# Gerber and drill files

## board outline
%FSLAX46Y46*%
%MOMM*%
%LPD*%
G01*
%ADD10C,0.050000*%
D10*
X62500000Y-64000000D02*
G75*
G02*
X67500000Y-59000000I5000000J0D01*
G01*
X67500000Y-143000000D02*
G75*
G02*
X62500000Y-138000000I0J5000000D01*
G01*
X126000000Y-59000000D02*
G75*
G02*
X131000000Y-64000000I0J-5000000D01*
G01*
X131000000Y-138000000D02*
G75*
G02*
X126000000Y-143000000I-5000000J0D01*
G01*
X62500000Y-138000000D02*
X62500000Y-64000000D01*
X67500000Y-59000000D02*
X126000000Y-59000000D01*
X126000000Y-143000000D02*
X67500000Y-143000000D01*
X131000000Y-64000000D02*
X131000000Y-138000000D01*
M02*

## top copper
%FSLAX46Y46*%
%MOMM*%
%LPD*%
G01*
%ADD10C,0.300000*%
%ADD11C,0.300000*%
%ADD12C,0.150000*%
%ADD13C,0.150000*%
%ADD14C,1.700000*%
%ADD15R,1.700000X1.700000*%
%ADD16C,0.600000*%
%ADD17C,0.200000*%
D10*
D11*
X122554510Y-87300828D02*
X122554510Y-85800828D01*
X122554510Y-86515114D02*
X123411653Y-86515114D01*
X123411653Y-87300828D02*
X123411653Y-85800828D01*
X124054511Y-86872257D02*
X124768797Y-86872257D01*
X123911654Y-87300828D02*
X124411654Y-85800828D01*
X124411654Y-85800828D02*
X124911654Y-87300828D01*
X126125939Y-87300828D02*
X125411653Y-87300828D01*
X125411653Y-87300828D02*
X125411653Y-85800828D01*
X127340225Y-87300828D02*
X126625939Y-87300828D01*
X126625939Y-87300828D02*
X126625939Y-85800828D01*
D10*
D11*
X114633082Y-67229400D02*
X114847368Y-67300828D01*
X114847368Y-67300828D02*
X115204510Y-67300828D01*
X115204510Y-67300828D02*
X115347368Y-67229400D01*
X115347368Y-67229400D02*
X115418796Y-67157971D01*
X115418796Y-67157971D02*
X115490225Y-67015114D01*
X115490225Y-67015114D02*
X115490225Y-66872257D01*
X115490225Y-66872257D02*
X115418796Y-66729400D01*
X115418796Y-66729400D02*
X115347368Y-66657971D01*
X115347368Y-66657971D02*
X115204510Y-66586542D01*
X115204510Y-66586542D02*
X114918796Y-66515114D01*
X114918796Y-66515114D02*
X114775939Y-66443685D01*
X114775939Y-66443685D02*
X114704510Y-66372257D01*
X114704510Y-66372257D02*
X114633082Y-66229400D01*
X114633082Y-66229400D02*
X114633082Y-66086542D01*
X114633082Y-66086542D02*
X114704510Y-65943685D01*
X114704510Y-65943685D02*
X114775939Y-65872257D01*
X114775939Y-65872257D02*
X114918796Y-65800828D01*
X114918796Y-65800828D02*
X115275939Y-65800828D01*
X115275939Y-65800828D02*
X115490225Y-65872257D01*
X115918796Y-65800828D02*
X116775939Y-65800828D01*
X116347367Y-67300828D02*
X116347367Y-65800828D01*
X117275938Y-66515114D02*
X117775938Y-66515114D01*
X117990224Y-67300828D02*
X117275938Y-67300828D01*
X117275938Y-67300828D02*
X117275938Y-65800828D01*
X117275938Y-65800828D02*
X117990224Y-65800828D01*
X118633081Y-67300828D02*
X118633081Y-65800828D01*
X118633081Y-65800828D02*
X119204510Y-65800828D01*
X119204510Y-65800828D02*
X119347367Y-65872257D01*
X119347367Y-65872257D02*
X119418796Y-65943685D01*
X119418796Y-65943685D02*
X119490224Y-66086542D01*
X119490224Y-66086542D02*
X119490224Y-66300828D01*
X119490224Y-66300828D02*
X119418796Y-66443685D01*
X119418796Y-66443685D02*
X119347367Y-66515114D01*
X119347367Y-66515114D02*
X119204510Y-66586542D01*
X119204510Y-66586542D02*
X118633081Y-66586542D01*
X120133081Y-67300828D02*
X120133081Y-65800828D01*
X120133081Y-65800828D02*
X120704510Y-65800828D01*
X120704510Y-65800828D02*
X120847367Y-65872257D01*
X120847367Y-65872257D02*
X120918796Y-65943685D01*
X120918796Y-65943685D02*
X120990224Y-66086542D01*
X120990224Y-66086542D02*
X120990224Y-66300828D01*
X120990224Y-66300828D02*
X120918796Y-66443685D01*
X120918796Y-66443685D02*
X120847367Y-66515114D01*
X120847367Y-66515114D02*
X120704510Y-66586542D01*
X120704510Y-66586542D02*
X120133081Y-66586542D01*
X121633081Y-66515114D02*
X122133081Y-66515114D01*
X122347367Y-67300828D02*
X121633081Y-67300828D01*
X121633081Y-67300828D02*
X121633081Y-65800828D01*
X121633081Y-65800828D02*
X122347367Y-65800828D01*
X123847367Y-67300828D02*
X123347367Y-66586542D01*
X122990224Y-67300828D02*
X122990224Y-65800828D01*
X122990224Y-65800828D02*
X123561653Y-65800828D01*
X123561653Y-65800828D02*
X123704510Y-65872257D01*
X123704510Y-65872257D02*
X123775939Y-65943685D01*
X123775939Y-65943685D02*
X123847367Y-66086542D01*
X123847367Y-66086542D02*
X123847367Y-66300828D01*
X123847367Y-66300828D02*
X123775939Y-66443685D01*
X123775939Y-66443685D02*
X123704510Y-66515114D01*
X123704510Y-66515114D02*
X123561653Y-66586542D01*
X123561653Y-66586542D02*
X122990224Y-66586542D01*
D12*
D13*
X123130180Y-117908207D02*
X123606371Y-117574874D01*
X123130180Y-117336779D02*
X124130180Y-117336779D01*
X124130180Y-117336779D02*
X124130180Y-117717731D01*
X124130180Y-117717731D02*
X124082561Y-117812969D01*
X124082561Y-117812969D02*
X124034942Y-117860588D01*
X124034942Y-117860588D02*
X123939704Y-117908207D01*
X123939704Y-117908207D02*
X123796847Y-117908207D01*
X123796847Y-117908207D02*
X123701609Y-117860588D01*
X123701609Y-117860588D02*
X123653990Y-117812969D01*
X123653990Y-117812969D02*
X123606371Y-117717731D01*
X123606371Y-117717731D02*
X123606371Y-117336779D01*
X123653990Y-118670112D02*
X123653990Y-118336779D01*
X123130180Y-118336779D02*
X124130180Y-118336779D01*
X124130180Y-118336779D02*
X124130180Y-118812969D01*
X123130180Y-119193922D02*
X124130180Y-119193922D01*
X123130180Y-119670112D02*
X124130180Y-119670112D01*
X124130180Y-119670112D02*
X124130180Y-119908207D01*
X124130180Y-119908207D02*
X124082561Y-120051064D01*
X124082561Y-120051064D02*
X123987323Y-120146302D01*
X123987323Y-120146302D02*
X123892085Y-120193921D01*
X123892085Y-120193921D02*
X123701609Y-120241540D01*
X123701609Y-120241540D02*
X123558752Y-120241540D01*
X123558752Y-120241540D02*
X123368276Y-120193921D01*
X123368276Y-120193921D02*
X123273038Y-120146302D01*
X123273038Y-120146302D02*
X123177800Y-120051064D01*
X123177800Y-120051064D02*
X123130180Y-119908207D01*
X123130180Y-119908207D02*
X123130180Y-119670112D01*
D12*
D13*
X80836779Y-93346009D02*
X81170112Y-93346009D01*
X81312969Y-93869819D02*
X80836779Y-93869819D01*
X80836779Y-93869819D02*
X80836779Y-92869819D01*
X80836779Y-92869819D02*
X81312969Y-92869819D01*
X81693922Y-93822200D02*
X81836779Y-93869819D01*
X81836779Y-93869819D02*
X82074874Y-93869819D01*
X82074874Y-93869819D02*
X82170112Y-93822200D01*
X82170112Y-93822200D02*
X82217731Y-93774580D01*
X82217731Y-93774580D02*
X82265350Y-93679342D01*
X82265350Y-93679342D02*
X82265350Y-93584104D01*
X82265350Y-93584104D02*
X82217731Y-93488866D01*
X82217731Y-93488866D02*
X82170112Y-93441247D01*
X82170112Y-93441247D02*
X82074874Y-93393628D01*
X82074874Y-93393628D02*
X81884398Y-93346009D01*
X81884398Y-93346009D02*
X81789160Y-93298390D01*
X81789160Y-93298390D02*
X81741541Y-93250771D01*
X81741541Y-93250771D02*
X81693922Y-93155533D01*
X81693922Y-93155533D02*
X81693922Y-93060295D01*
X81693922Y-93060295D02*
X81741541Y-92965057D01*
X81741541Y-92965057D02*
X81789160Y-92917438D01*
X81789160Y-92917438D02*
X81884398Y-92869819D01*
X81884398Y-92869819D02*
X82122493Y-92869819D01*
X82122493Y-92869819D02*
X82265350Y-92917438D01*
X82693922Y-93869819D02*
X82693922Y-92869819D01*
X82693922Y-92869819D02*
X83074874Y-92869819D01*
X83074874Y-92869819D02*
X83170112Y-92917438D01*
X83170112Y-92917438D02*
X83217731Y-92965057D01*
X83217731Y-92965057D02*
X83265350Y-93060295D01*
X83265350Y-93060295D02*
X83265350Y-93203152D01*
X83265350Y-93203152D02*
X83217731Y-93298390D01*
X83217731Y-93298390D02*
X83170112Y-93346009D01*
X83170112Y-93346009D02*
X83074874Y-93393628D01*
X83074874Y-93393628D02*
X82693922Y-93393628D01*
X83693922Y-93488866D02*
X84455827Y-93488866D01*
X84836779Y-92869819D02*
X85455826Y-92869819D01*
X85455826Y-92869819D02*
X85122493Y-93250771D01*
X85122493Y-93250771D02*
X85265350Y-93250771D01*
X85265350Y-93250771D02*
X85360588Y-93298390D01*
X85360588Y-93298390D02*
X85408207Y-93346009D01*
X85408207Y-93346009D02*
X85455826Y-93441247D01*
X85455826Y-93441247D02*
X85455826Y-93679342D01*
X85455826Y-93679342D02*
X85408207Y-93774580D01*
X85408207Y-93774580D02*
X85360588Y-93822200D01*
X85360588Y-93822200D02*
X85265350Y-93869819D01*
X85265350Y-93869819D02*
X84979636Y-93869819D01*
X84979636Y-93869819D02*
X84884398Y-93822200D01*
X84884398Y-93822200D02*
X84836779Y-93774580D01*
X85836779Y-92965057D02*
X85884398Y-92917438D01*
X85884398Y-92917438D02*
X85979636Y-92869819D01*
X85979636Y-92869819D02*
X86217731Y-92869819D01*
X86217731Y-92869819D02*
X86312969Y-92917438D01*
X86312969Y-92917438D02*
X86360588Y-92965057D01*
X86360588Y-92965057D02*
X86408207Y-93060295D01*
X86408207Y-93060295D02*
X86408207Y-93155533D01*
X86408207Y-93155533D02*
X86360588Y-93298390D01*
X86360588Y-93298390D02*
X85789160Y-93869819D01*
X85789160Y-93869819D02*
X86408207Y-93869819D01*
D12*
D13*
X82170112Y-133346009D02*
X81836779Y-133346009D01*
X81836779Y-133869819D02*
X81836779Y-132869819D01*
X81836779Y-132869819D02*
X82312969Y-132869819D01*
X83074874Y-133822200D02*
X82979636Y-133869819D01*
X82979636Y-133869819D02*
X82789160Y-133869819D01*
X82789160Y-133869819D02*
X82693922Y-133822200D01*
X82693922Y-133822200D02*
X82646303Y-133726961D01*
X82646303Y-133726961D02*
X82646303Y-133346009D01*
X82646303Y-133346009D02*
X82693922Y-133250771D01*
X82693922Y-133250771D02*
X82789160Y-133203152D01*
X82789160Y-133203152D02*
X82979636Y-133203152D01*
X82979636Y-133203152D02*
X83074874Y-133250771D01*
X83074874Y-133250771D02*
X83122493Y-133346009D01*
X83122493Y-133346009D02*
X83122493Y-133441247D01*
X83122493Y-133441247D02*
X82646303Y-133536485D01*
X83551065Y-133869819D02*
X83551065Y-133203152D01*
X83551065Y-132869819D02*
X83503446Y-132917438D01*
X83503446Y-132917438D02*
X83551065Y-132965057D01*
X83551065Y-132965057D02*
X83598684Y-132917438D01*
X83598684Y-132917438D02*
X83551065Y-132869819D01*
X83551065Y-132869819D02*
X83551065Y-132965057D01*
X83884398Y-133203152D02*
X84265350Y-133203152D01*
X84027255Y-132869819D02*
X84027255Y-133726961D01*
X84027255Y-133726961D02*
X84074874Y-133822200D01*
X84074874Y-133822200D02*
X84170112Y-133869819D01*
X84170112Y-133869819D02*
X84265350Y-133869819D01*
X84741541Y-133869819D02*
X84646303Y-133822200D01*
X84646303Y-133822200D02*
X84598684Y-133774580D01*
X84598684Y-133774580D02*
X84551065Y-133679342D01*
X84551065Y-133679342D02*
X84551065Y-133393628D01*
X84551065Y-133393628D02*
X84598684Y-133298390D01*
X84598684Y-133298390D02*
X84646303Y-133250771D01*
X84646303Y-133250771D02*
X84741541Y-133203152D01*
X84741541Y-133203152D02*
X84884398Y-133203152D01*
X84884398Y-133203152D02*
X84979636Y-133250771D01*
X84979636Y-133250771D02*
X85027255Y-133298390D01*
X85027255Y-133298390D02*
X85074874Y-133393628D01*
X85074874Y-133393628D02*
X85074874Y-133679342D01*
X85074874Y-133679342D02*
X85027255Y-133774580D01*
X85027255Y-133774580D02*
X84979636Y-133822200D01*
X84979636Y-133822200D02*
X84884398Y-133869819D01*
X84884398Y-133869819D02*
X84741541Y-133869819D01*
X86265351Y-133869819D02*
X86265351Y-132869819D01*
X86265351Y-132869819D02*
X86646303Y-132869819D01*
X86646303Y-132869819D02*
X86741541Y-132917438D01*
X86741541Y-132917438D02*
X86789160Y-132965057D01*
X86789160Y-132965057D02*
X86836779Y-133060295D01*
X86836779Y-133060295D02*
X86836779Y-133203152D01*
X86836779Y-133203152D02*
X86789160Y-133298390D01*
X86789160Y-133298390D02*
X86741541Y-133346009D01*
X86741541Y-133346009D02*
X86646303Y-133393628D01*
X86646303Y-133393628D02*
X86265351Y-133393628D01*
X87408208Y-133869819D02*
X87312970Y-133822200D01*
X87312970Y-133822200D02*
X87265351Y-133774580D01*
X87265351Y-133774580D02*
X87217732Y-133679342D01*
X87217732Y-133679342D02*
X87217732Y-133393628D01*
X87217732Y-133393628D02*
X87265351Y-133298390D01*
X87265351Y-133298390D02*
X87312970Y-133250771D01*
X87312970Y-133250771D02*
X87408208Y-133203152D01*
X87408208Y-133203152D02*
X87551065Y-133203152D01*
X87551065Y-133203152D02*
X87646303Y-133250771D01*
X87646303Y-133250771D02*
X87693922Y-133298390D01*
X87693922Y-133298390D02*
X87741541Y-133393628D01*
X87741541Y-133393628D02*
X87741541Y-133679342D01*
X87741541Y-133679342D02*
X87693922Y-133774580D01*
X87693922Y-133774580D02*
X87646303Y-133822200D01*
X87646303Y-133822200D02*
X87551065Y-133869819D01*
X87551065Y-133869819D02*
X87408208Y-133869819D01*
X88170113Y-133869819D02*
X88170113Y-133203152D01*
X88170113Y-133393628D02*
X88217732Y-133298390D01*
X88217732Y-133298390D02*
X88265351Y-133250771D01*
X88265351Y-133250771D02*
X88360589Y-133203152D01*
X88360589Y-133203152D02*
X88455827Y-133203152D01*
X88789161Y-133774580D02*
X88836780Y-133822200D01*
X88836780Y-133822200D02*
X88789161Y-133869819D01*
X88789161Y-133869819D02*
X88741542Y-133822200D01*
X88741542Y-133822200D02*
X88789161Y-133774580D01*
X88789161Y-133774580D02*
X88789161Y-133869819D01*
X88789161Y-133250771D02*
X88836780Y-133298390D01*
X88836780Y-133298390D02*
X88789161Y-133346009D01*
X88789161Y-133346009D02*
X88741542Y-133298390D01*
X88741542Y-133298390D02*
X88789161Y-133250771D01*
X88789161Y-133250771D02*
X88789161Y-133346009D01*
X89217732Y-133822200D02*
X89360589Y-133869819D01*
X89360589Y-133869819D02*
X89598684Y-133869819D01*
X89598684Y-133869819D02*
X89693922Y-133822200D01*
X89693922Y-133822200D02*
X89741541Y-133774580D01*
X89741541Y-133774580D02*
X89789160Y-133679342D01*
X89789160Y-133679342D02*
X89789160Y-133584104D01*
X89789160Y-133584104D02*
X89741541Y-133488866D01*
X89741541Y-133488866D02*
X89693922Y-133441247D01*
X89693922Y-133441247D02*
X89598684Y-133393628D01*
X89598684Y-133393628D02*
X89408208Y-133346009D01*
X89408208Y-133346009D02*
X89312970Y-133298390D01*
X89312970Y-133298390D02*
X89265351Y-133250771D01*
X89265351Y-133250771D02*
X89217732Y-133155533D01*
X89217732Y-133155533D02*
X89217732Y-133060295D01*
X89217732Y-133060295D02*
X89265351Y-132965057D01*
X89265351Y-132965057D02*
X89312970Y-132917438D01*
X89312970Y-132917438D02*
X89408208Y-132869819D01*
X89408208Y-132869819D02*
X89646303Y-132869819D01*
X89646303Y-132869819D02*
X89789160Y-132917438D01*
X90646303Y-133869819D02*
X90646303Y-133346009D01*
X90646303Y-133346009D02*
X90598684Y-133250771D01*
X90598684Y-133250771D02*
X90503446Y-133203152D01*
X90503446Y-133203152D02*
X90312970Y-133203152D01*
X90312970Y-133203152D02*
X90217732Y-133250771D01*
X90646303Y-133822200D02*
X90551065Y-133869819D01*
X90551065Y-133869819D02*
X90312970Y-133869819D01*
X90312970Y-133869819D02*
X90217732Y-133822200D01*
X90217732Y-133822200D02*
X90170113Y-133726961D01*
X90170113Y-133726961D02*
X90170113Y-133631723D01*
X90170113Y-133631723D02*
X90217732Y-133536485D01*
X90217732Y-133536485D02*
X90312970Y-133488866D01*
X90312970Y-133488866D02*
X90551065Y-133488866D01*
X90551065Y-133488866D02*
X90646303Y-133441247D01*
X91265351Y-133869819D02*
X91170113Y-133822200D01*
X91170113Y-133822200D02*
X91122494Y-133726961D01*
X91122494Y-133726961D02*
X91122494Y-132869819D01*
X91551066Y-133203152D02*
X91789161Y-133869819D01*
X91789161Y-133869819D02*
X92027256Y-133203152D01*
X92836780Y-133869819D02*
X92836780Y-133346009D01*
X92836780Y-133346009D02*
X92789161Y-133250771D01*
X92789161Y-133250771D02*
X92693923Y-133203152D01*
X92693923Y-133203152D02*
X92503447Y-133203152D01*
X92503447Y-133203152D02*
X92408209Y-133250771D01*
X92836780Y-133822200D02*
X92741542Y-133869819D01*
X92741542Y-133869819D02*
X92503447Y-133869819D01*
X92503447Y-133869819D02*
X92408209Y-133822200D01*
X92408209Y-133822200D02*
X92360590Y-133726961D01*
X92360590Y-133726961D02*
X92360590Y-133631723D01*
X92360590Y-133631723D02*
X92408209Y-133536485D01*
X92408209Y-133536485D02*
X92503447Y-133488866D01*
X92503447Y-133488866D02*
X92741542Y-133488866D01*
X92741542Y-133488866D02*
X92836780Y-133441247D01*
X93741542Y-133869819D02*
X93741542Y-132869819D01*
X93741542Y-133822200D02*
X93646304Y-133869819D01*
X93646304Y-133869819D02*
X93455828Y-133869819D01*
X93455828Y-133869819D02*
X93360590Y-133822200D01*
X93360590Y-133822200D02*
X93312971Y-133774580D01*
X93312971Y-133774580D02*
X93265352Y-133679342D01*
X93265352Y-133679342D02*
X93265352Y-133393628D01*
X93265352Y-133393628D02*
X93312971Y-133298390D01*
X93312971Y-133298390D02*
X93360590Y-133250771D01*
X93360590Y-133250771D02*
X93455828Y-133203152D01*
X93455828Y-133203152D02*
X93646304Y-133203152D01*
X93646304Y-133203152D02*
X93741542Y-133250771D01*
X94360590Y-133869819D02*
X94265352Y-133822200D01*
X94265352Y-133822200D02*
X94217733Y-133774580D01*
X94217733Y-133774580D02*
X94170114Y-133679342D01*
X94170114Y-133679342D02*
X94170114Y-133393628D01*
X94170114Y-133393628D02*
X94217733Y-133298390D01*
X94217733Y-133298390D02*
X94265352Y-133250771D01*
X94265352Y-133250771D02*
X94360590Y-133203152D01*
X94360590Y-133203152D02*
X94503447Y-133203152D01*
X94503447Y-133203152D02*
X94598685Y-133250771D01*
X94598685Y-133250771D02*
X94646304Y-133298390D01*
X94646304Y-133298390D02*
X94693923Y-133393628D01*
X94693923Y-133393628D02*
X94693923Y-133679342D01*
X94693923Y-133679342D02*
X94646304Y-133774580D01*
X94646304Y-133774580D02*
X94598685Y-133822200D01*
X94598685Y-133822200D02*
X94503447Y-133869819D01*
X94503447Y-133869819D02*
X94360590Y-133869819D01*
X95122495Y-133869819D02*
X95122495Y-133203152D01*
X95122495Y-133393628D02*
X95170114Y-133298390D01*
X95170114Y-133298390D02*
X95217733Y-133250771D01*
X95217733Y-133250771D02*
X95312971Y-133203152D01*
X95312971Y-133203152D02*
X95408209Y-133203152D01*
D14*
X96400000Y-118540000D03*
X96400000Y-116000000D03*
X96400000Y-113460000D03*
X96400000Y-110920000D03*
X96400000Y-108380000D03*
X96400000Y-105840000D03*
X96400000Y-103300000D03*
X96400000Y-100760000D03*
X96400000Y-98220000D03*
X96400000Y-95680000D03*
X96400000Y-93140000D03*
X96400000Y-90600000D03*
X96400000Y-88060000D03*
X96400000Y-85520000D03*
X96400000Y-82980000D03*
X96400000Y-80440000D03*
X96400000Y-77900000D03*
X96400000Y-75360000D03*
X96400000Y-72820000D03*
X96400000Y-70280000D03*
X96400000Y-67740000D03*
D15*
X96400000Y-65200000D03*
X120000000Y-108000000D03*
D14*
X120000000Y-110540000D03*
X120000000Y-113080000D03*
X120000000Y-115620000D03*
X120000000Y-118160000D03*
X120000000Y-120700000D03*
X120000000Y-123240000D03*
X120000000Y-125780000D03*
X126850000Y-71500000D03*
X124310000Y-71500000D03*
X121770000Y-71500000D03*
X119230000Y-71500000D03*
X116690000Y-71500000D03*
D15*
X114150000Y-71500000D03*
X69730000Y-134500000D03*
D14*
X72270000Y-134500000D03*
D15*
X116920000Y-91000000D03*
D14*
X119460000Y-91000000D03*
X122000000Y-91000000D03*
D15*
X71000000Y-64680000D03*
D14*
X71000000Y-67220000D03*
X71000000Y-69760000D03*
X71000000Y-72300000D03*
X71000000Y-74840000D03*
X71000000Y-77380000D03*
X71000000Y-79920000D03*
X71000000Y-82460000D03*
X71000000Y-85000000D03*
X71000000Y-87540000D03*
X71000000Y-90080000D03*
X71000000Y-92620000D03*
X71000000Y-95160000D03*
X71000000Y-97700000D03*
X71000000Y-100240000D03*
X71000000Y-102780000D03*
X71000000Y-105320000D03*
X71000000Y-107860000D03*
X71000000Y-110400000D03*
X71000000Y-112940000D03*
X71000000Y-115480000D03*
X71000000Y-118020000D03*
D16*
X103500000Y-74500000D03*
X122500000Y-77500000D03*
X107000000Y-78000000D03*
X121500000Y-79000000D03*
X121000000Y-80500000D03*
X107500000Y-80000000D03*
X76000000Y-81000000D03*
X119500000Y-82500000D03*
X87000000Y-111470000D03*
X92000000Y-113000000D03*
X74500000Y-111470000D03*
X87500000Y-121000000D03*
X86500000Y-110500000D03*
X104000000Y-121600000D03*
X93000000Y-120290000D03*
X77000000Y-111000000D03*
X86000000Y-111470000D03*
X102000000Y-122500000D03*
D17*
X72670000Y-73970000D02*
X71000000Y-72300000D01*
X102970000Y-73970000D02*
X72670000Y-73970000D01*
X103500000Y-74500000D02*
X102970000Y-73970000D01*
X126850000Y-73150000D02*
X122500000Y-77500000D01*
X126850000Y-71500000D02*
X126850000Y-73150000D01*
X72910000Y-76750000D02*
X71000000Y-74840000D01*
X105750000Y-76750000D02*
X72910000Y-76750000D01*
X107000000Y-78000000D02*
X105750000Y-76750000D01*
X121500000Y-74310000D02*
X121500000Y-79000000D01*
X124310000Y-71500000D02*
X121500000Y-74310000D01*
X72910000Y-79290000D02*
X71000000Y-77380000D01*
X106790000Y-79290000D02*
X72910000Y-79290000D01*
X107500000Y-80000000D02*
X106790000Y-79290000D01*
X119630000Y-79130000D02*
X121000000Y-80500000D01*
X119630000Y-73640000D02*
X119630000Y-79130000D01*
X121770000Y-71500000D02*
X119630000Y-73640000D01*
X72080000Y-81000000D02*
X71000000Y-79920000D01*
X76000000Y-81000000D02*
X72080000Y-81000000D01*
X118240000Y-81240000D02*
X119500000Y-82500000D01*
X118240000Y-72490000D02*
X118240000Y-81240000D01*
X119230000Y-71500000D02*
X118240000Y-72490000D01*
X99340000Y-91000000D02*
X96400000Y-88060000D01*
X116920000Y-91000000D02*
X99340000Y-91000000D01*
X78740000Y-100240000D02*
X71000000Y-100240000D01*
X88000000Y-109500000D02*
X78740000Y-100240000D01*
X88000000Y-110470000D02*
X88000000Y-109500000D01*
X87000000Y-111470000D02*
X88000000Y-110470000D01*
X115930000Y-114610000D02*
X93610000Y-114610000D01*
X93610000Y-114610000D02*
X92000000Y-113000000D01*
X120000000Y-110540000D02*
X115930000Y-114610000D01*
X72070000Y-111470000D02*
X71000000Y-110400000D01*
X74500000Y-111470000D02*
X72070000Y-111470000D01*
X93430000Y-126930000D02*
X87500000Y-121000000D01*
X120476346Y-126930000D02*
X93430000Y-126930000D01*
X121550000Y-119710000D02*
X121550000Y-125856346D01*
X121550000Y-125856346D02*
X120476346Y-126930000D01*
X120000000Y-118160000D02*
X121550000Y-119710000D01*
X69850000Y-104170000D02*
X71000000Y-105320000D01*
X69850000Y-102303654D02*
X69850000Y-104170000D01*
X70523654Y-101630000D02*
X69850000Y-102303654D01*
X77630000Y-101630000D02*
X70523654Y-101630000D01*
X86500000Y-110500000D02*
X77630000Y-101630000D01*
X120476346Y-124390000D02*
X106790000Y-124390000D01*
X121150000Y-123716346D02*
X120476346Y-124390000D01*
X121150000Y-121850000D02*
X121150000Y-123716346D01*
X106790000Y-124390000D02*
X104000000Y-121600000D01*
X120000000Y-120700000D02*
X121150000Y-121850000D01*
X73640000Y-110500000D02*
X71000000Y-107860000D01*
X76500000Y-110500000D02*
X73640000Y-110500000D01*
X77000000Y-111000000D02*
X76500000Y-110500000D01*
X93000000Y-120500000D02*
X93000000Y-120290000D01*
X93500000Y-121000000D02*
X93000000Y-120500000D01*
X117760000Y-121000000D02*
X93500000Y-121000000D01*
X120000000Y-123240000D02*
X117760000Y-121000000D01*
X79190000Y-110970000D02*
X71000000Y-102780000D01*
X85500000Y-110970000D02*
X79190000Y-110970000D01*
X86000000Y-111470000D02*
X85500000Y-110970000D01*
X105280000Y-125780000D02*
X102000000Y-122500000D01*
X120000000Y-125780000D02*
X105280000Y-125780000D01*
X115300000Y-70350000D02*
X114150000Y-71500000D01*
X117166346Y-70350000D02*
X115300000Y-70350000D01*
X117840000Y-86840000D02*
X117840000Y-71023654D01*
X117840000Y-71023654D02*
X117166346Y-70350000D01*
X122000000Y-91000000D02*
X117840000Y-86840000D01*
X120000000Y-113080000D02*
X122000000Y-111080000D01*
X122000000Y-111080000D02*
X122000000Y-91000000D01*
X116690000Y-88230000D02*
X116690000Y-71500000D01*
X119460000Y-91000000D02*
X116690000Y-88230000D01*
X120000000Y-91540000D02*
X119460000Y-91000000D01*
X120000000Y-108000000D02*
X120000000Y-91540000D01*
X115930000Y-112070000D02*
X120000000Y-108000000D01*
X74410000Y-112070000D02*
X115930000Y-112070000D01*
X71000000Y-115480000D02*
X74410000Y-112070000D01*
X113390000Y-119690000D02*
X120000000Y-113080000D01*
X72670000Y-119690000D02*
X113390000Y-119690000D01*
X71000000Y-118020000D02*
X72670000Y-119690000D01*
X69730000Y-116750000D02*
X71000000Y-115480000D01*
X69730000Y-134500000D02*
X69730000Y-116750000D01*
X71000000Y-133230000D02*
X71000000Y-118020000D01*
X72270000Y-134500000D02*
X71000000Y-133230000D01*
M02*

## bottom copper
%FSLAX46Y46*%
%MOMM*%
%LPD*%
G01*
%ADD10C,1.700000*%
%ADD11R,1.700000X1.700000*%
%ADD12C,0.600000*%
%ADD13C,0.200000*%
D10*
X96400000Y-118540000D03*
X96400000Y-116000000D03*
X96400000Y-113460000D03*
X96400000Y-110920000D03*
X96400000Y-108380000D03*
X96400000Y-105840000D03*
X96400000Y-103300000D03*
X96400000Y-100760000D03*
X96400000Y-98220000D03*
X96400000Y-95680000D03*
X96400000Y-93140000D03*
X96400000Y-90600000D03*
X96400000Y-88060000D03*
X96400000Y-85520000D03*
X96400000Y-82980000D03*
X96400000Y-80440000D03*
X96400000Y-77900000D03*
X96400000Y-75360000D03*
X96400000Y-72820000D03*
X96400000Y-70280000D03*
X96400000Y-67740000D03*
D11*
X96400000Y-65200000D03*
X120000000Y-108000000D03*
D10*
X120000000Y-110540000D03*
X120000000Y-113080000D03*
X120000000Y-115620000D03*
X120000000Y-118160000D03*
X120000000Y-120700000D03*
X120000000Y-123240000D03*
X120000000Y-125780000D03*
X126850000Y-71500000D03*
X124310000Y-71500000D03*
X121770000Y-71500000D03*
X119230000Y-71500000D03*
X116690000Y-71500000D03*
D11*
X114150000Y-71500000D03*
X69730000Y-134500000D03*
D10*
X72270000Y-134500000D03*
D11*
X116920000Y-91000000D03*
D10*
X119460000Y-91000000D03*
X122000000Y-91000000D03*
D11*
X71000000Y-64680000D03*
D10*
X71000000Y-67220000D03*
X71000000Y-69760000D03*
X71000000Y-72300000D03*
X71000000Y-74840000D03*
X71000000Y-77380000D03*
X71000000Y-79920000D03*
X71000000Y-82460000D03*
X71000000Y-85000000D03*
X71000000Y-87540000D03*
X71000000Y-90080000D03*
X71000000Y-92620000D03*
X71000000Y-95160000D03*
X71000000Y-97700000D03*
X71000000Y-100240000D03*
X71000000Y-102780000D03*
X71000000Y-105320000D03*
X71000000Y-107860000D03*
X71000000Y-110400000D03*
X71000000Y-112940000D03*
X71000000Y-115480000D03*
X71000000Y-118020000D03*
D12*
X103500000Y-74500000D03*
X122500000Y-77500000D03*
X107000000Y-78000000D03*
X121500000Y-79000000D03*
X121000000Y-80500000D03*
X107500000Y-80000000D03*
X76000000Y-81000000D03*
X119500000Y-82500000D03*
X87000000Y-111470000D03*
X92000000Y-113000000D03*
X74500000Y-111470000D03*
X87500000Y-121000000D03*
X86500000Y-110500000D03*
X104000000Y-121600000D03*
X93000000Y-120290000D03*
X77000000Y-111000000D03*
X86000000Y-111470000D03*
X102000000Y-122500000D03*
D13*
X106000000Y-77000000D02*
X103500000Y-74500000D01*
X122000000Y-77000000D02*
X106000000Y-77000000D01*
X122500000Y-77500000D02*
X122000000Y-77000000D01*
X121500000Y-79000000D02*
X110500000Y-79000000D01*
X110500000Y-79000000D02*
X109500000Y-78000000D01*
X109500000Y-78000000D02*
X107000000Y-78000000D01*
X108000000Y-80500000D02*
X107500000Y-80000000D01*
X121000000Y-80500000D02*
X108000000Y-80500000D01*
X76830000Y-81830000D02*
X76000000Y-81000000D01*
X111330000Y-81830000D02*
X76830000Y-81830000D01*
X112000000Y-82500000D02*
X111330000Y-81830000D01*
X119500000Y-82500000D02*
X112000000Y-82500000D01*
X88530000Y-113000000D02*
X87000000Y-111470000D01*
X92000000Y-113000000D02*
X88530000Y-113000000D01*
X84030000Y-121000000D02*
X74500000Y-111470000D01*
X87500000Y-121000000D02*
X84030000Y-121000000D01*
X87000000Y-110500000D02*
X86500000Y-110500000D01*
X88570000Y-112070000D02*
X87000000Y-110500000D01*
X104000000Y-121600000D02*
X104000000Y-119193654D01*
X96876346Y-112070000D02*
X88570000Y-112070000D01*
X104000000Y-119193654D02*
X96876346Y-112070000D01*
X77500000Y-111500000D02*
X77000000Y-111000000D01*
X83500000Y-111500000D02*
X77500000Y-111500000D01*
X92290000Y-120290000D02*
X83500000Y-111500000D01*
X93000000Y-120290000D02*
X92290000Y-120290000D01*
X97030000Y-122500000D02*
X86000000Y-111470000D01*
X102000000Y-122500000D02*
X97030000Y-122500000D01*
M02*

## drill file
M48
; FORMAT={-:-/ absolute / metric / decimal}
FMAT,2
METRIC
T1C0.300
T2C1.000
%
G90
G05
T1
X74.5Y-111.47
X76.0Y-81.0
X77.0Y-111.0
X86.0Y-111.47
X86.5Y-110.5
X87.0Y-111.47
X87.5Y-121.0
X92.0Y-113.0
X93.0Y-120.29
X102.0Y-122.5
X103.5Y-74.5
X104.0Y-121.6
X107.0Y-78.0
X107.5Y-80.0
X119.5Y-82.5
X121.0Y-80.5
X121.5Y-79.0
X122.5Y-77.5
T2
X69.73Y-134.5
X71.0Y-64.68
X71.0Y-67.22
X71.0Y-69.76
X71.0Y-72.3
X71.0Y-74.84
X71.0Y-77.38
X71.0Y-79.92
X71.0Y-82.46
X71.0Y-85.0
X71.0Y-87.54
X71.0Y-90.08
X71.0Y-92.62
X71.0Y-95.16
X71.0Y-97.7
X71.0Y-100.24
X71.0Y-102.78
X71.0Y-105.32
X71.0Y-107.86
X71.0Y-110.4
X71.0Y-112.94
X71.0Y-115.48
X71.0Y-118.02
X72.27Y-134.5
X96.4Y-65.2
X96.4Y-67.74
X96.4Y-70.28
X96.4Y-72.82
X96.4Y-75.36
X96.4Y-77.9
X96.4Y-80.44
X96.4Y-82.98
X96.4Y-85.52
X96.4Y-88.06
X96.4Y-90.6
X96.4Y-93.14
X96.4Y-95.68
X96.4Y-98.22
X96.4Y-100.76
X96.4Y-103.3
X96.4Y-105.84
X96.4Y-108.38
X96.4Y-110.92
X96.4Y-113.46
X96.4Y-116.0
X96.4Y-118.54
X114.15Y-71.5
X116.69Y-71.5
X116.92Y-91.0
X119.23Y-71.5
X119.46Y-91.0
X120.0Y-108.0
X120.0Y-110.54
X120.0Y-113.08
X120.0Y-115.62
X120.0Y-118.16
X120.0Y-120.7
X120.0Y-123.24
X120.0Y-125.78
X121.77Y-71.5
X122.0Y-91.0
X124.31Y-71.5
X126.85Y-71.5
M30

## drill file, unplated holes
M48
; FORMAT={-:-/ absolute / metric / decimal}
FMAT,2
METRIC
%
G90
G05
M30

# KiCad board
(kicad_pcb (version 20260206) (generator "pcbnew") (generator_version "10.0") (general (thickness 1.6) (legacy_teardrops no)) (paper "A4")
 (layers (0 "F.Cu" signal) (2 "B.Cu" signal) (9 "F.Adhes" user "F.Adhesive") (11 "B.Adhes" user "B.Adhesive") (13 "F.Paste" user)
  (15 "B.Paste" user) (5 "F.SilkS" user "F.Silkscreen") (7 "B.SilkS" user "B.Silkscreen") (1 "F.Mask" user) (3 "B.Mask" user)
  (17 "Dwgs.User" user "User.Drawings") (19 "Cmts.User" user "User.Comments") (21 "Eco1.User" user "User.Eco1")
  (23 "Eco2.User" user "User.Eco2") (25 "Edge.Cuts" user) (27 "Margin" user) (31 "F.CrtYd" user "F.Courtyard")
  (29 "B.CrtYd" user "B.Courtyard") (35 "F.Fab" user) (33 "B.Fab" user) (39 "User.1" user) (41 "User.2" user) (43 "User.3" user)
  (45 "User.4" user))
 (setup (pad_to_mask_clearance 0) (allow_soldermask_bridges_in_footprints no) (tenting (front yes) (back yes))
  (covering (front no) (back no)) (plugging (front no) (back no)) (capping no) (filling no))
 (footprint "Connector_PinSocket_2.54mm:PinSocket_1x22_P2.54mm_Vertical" (layer "F.Cu") (at 96.4 65.2)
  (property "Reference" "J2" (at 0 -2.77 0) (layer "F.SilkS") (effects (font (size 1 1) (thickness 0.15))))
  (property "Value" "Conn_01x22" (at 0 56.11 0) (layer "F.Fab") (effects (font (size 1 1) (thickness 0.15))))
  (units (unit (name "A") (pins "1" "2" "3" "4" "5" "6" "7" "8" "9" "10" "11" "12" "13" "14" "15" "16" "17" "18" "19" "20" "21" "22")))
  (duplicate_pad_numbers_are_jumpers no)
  (pad "1" thru_hole rect (at 0 0) (size 1.7 1.7) (drill 1) (layers "*.Cu" "*.Mask") (remove_unused_layers no)
   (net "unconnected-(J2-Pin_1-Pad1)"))
  (pad "2" thru_hole circle (at 0 2.54) (size 1.7 1.7) (drill 1) (layers "*.Cu" "*.Mask") (remove_unused_layers no)
   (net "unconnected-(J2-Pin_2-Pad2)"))
  (pad "3" thru_hole circle (at 0 5.08) (size 1.7 1.7) (drill 1) (layers "*.Cu" "*.Mask") (remove_unused_layers no)
   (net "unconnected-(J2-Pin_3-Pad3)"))
  (pad "4" thru_hole circle (at 0 7.62) (size 1.7 1.7) (drill 1) (layers "*.Cu" "*.Mask") (remove_unused_layers no)
   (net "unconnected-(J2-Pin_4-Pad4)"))
  (pad "5" thru_hole circle (at 0 10.16) (size 1.7 1.7) (drill 1) (layers "*.Cu" "*.Mask") (remove_unused_layers no)
   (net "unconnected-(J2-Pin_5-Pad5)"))
  (pad "6" thru_hole circle (at 0 12.7) (size 1.7 1.7) (drill 1) (layers "*.Cu" "*.Mask") (remove_unused_layers no)
   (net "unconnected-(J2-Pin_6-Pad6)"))
  (pad "7" thru_hole circle (at 0 15.24) (size 1.7 1.7) (drill 1) (layers "*.Cu" "*.Mask") (remove_unused_layers no)
   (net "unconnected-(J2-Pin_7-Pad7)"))
  (pad "8" thru_hole circle (at 0 17.78) (size 1.7 1.7) (drill 1) (layers "*.Cu" "*.Mask") (remove_unused_layers no)
   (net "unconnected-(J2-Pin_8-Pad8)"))
  (pad "9" thru_hole circle (at 0 20.32) (size 1.7 1.7) (drill 1) (layers "*.Cu" "*.Mask") (remove_unused_layers no)
   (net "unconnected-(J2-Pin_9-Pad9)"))
  (pad "10" thru_hole circle (at 0 22.86) (size 1.7 1.7) (drill 1) (layers "*.Cu" "*.Mask") (remove_unused_layers no)
   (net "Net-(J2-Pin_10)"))
  (pad "11" thru_hole circle (at 0 25.4) (size 1.7 1.7) (drill 1) (layers "*.Cu" "*.Mask") (remove_unused_layers no)
   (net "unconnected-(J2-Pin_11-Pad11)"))
  (pad "12" thru_hole circle (at 0 27.94) (size 1.7 1.7) (drill 1) (layers "*.Cu" "*.Mask") (remove_unused_layers no)
   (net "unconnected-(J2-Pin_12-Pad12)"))
  (pad "13" thru_hole circle (at 0 30.48) (size 1.7 1.7) (drill 1) (layers "*.Cu" "*.Mask") (remove_unused_layers no)
   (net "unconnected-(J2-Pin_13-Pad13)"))
  (pad "14" thru_hole circle (at 0 33.02) (size 1.7 1.7) (drill 1) (layers "*.Cu" "*.Mask") (remove_unused_layers no)
   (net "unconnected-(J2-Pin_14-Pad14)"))
  (pad "15" thru_hole circle (at 0 35.56) (size 1.7 1.7) (drill 1) (layers "*.Cu" "*.Mask") (remove_unused_layers no)
   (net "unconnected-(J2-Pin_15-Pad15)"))
  (pad "16" thru_hole circle (at 0 38.1) (size 1.7 1.7) (drill 1) (layers "*.Cu" "*.Mask") (remove_unused_layers no)
   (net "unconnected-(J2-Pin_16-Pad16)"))
  (pad "17" thru_hole circle (at 0 40.64) (size 1.7 1.7) (drill 1) (layers "*.Cu" "*.Mask") (remove_unused_layers no)
   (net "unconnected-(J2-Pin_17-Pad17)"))
  (pad "18" thru_hole circle (at 0 43.18) (size 1.7 1.7) (drill 1) (layers "*.Cu" "*.Mask") (remove_unused_layers no)
   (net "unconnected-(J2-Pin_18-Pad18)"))
  (pad "19" thru_hole circle (at 0 45.72) (size 1.7 1.7) (drill 1) (layers "*.Cu" "*.Mask") (remove_unused_layers no)
   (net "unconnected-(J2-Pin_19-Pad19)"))
  (pad "20" thru_hole circle (at 0 48.26) (size 1.7 1.7) (drill 1) (layers "*.Cu" "*.Mask") (remove_unused_layers no)
   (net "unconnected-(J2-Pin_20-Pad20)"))
  (pad "21" thru_hole circle (at 0 50.8) (size 1.7 1.7) (drill 1) (layers "*.Cu" "*.Mask") (remove_unused_layers no)
   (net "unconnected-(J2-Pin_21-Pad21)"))
  (pad "22" thru_hole circle (at 0 53.34) (size 1.7 1.7) (drill 1) (layers "*.Cu" "*.Mask") (remove_unused_layers no)
   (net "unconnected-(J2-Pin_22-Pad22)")))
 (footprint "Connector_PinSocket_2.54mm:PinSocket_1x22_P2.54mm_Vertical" (layer "F.Cu") (at 71 64.68)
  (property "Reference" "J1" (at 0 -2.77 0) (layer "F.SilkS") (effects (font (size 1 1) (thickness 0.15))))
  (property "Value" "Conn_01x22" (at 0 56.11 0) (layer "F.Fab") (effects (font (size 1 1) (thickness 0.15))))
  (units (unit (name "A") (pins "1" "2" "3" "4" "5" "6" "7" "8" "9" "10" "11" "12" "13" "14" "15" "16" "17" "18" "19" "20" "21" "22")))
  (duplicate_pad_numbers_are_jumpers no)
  (pad "1" thru_hole rect (at 0 0) (size 1.7 1.7) (drill 1) (layers "*.Cu" "*.Mask") (remove_unused_layers no)
   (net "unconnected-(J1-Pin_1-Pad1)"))
  (pad "2" thru_hole circle (at 0 2.54) (size 1.7 1.7) (drill 1) (layers "*.Cu" "*.Mask") (remove_unused_layers no)
   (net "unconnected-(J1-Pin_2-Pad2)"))
  (pad "3" thru_hole circle (at 0 5.08) (size 1.7 1.7) (drill 1) (layers "*.Cu" "*.Mask") (remove_unused_layers no)
   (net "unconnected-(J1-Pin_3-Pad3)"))
  (pad "4" thru_hole circle (at 0 7.62) (size 1.7 1.7) (drill 1) (layers "*.Cu" "*.Mask") (remove_unused_layers no) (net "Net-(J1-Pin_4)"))
  (pad "5" thru_hole circle (at 0 10.16) (size 1.7 1.7) (drill 1) (layers "*.Cu" "*.Mask") (remove_unused_layers no) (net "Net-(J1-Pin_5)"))
  (pad "6" thru_hole circle (at 0 12.7) (size 1.7 1.7) (drill 1) (layers "*.Cu" "*.Mask") (remove_unused_layers no) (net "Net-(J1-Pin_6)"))
  (pad "7" thru_hole circle (at 0 15.24) (size 1.7 1.7) (drill 1) (layers "*.Cu" "*.Mask") (remove_unused_layers no) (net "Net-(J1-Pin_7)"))
  (pad "8" thru_hole circle (at 0 17.78) (size 1.7 1.7) (drill 1) (layers "*.Cu" "*.Mask") (remove_unused_layers no)
   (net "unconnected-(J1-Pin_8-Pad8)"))
  (pad "9" thru_hole circle (at 0 20.32) (size 1.7 1.7) (drill 1) (layers "*.Cu" "*.Mask") (remove_unused_layers no)
   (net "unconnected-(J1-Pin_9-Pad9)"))
  (pad "10" thru_hole circle (at 0 22.86) (size 1.7 1.7) (drill 1) (layers "*.Cu" "*.Mask") (remove_unused_layers no)
   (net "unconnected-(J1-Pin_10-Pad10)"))
  (pad "11" thru_hole circle (at 0 25.4) (size 1.7 1.7) (drill 1) (layers "*.Cu" "*.Mask") (remove_unused_layers no)
   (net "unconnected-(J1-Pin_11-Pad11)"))
  (pad "12" thru_hole circle (at 0 27.94) (size 1.7 1.7) (drill 1) (layers "*.Cu" "*.Mask") (remove_unused_layers no)
   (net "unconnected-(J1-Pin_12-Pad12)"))
  (pad "13" thru_hole circle (at 0 30.48) (size 1.7 1.7) (drill 1) (layers "*.Cu" "*.Mask") (remove_unused_layers no)
   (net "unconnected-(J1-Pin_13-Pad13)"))
  (pad "14" thru_hole circle (at 0 33.02) (size 1.7 1.7) (drill 1) (layers "*.Cu" "*.Mask") (remove_unused_layers no)
   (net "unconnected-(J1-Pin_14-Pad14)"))
  (pad "15" thru_hole circle (at 0 35.56) (size 1.7 1.7) (drill 1) (layers "*.Cu" "*.Mask") (remove_unused_layers no)
   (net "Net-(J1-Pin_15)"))
  (pad "16" thru_hole circle (at 0 38.1) (size 1.7 1.7) (drill 1) (layers "*.Cu" "*.Mask") (remove_unused_layers no) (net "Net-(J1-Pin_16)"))
  (pad "17" thru_hole circle (at 0 40.64) (size 1.7 1.7) (drill 1) (layers "*.Cu" "*.Mask") (remove_unused_layers no)
   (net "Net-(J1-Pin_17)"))
  (pad "18" thru_hole circle (at 0 43.18) (size 1.7 1.7) (drill 1) (layers "*.Cu" "*.Mask") (remove_unused_layers no)
   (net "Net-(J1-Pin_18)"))
  (pad "19" thru_hole circle (at 0 45.72) (size 1.7 1.7) (drill 1) (layers "*.Cu" "*.Mask") (remove_unused_layers no)
   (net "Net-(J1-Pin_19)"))
  (pad "20" thru_hole circle (at 0 48.26) (size 1.7 1.7) (drill 1) (layers "*.Cu" "*.Mask") (remove_unused_layers no)
   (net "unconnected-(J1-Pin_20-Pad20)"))
  (pad "21" thru_hole circle (at 0 50.8) (size 1.7 1.7) (drill 1) (layers "*.Cu" "*.Mask") (remove_unused_layers no) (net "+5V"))
  (pad "22" thru_hole circle (at 0 53.34) (size 1.7 1.7) (drill 1) (layers "*.Cu" "*.Mask") (remove_unused_layers no) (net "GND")))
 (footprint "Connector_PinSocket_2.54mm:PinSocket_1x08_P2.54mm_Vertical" (layer "F.Cu") (at 120 108)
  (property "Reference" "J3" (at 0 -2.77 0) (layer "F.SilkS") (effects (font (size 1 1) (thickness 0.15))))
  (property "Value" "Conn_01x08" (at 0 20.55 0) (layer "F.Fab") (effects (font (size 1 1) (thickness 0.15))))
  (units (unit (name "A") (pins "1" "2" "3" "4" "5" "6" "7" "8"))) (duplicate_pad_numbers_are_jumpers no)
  (pad "1" thru_hole rect (at 0 0) (size 1.7 1.7) (drill 1) (layers "*.Cu" "*.Mask") (remove_unused_layers no) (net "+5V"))
  (pad "2" thru_hole circle (at 0 2.54) (size 1.7 1.7) (drill 1) (layers "*.Cu" "*.Mask") (remove_unused_layers no) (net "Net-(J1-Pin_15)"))
  (pad "3" thru_hole circle (at 0 5.08) (size 1.7 1.7) (drill 1) (layers "*.Cu" "*.Mask") (remove_unused_layers no) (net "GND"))
  (pad "4" thru_hole circle (at 0 7.62) (size 1.7 1.7) (drill 1) (layers "*.Cu" "*.Mask") (remove_unused_layers no)
   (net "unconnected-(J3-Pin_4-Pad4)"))
  (pad "5" thru_hole circle (at 0 10.16) (size 1.7 1.7) (drill 1) (layers "*.Cu" "*.Mask") (remove_unused_layers no) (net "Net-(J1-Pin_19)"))
  (pad "6" thru_hole circle (at 0 12.7) (size 1.7 1.7) (drill 1) (layers "*.Cu" "*.Mask") (remove_unused_layers no) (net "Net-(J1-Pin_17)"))
  (pad "7" thru_hole circle (at 0 15.24) (size 1.7 1.7) (drill 1) (layers "*.Cu" "*.Mask") (remove_unused_layers no) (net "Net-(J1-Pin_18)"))
  (pad "8" thru_hole circle (at 0 17.78) (size 1.7 1.7) (drill 1) (layers "*.Cu" "*.Mask") (remove_unused_layers no) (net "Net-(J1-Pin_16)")))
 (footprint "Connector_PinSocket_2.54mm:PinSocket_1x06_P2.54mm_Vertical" (layer "F.Cu") (at 114.15 71.5 90)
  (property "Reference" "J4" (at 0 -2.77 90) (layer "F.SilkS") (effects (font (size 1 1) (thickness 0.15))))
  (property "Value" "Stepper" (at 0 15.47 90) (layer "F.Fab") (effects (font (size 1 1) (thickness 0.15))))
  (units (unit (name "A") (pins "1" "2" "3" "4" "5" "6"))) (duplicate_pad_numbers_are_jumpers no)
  (pad "1" thru_hole rect (at 0 0 90) (size 1.7 1.7) (drill 1) (layers "*.Cu" "*.Mask") (remove_unused_layers no) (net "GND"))
  (pad "2" thru_hole circle (at 0 2.54 90) (size 1.7 1.7) (drill 1) (layers "*.Cu" "*.Mask") (remove_unused_layers no) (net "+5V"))
  (pad "3" thru_hole circle (at 0 5.08 90) (size 1.7 1.7) (drill 1) (layers "*.Cu" "*.Mask") (remove_unused_layers no)
   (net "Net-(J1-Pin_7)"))
  (pad "4" thru_hole circle (at 0 7.62 90) (size 1.7 1.7) (drill 1) (layers "*.Cu" "*.Mask") (remove_unused_layers no)
   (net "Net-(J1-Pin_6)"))
  (pad "5" thru_hole circle (at 0 10.16 90) (size 1.7 1.7) (drill 1) (layers "*.Cu" "*.Mask") (remove_unused_layers no)
   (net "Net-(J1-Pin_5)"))
  (pad "6" thru_hole circle (at 0 12.7 90) (size 1.7 1.7) (drill 1) (layers "*.Cu" "*.Mask") (remove_unused_layers no)
   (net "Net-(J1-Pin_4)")))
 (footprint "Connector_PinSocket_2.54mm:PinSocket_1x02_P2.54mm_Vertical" (layer "F.Cu") (at 69.73 134.5 90)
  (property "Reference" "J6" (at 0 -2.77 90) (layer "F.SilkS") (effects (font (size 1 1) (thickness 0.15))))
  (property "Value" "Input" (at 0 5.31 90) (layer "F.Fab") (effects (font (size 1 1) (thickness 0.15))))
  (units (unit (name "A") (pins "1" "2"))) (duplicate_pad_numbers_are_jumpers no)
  (pad "1" thru_hole rect (at 0 0 90) (size 1.7 1.7) (drill 1) (layers "*.Cu" "*.Mask") (remove_unused_layers no) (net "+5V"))
  (pad "2" thru_hole circle (at 0 2.54 90) (size 1.7 1.7) (drill 1) (layers "*.Cu" "*.Mask") (remove_unused_layers no) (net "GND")))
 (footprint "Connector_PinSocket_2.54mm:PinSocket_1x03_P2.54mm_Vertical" (layer "F.Cu") (at 116.92 91 90)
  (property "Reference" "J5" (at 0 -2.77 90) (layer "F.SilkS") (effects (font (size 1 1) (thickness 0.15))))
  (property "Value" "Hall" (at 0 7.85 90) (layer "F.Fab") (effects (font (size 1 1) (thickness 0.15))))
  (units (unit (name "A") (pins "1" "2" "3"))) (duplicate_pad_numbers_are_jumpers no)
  (pad "1" thru_hole rect (at 0 0 90) (size 1.7 1.7) (drill 1) (layers "*.Cu" "*.Mask") (remove_unused_layers no) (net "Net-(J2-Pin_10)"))
  (pad "2" thru_hole circle (at 0 2.54 90) (size 1.7 1.7) (drill 1) (layers "*.Cu" "*.Mask") (remove_unused_layers no) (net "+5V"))
  (pad "3" thru_hole circle (at 0 5.08 90) (size 1.7 1.7) (drill 1) (layers "*.Cu" "*.Mask") (remove_unused_layers no) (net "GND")))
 (gr_arc (start 62.5 64) (mid 63.964466 60.464466) (end 67.5 59) (stroke (width 0.05) (type default)) (layer "Edge.Cuts"))
 (gr_line (start 62.5 138) (end 62.5 64) (stroke (width 0.05) (type default)) (layer "Edge.Cuts"))
 (gr_line (start 67.5 59) (end 126 59) (stroke (width 0.05) (type default)) (layer "Edge.Cuts"))
 (gr_arc (start 67.5 143) (mid 63.964466 141.535534) (end 62.5 138) (stroke (width 0.05) (type default)) (layer "Edge.Cuts"))
 (gr_arc (start 126 59) (mid 129.535534 60.464466) (end 131 64) (stroke (width 0.05) (type default)) (layer "Edge.Cuts"))
 (gr_line (start 126 143) (end 67.5 143) (stroke (width 0.05) (type default)) (layer "Edge.Cuts"))
 (gr_line (start 131 64) (end 131 138) (stroke (width 0.05) (type default)) (layer "Edge.Cuts"))
 (gr_arc (start 131 138) (mid 129.535534 141.535534) (end 126 143) (stroke (width 0.05) (type default)) (layer "Edge.Cuts"))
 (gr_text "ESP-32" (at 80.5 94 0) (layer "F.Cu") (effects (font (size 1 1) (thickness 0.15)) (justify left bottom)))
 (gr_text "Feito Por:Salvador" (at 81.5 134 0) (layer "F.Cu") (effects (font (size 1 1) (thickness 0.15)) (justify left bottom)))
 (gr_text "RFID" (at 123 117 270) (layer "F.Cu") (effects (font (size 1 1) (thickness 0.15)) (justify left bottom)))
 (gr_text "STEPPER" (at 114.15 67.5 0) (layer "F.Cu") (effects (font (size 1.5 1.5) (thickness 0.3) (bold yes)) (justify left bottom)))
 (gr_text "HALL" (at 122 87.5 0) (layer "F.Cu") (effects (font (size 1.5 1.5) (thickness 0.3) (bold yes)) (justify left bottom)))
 (segment (start 76.5 110.5) (end 73.64 110.5) (width 0.2) (layer "F.Cu") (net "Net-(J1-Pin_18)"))
 (segment (start 77 111) (end 76.5 110.5) (width 0.2) (layer "F.Cu") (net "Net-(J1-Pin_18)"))
 (segment (start 120 123.24) (end 117.76 121) (width 0.2) (layer "F.Cu") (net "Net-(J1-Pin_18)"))
 (segment (start 117.76 121) (end 93.5 121) (width 0.2) (layer "F.Cu") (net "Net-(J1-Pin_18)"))
 (segment (start 93 120.5) (end 93 120.29) (width 0.2) (layer "F.Cu") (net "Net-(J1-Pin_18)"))
 (segment (start 73.64 110.5) (end 71 107.86) (width 0.2) (layer "F.Cu") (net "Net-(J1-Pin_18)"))
 (segment (start 93.5 121) (end 93 120.5) (width 0.2) (layer "F.Cu") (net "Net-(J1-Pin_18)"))
 (via (at 77 111) (size 0.6) (drill 0.3) (layers "F.Cu" "B.Cu") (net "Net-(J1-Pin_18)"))
 (via (at 93 120.29) (size 0.6) (drill 0.3) (layers "F.Cu" "B.Cu") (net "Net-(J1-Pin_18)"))
 (segment (start 92.29 120.29) (end 83.5 111.5) (width 0.2) (layer "B.Cu") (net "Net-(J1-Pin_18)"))
 (segment (start 93 120.29) (end 92.29 120.29) (width 0.2) (layer "B.Cu") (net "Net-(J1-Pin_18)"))
 (segment (start 83.5 111.5) (end 77.5 111.5) (width 0.2) (layer "B.Cu") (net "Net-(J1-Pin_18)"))
 (segment (start 77.5 111.5) (end 77 111) (width 0.2) (layer "B.Cu") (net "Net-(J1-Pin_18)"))
 (segment (start 76 81) (end 72.08 81) (width 0.2) (layer "F.Cu") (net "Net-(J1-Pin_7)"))
 (segment (start 118.24 72.49) (end 118.24 81.24) (width 0.2) (layer "F.Cu") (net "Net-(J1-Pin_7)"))
 (segment (start 119.23 71.5) (end 118.24 72.49) (width 0.2) (layer "F.Cu") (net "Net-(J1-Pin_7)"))
 (segment (start 118.24 81.24) (end 119.5 82.5) (width 0.2) (layer "F.Cu") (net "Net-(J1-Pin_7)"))
 (segment (start 72.08 81) (end 71 79.92) (width 0.2) (layer "F.Cu") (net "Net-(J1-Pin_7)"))
 (via (at 76 81) (size 0.6) (drill 0.3) (layers "F.Cu" "B.Cu") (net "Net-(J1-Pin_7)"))
 (via (at 119.5 82.5) (size 0.6) (drill 0.3) (layers "F.Cu" "B.Cu") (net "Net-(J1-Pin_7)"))
 (segment (start 111.33 81.83) (end 76.83 81.83) (width 0.2) (layer "B.Cu") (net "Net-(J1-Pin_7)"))
 (segment (start 112 82.5) (end 111.33 81.83) (width 0.2) (layer "B.Cu") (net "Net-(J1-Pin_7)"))
 (segment (start 119.5 82.5) (end 112 82.5) (width 0.2) (layer "B.Cu") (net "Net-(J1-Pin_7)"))
 (segment (start 76.83 81.83) (end 76 81) (width 0.2) (layer "B.Cu") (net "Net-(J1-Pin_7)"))
 (segment (start 93.43 126.93) (end 87.5 121) (width 0.2) (layer "F.Cu") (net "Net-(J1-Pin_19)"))
 (segment (start 120 118.16) (end 121.55 119.71) (width 0.2) (layer "F.Cu") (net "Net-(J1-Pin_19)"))
 (segment (start 121.55 125.856346) (end 120.476346 126.93) (width 0.2) (layer "F.Cu") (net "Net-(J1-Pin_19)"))
 (segment (start 72.07 111.47) (end 71 110.4) (width 0.2) (layer "F.Cu") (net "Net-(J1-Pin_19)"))
 (segment (start 120.476346 126.93) (end 93.43 126.93) (width 0.2) (layer "F.Cu") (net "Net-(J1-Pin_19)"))
 (segment (start 121.55 119.71) (end 121.55 125.856346) (width 0.2) (layer "F.Cu") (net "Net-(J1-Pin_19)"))
 (segment (start 74.5 111.47) (end 72.07 111.47) (width 0.2) (layer "F.Cu") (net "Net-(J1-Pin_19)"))
 (via (at 74.5 111.47) (size 0.6) (drill 0.3) (layers "F.Cu" "B.Cu") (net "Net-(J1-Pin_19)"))
 (via (at 87.5 121) (size 0.6) (drill 0.3) (layers "F.Cu" "B.Cu") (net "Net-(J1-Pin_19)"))
 (segment (start 87.5 121) (end 84.03 121) (width 0.2) (layer "B.Cu") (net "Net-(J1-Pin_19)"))
 (segment (start 84.03 121) (end 74.5 111.47) (width 0.2) (layer "B.Cu") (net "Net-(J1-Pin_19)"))
 (segment (start 71 115.48) (end 74.41 112.07) (width 0.2) (layer "F.Cu") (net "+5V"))
 (segment (start 115.93 112.07) (end 120 108) (width 0.2) (layer "F.Cu") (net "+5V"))
 (segment (start 116.69 88.23) (end 116.69 71.5) (width 0.2) (layer "F.Cu") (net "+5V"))
 (segment (start 119.46 91) (end 116.69 88.23) (width 0.2) (layer "F.Cu") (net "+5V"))
 (segment (start 120 108) (end 120 91.54) (width 0.2) (layer "F.Cu") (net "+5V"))
 (segment (start 69.73 116.75) (end 71 115.48) (width 0.2) (layer "F.Cu") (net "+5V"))
 (segment (start 120 91.54) (end 119.46 91) (width 0.2) (layer "F.Cu") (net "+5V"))
 (segment (start 74.41 112.07) (end 115.93 112.07) (width 0.2) (layer "F.Cu") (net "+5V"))
 (segment (start 69.73 134.5) (end 69.73 116.75) (width 0.2) (layer "F.Cu") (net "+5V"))
 (segment (start 72.91 79.29) (end 71 77.38) (width 0.2) (layer "F.Cu") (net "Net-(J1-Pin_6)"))
 (segment (start 121.77 71.5) (end 119.63 73.64) (width 0.2) (layer "F.Cu") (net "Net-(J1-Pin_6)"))
 (segment (start 119.63 79.13) (end 121 80.5) (width 0.2) (layer "F.Cu") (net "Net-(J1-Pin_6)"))
 (segment (start 106.79 79.29) (end 72.91 79.29) (width 0.2) (layer "F.Cu") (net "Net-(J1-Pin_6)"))
 (segment (start 119.63 73.64) (end 119.63 79.13) (width 0.2) (layer "F.Cu") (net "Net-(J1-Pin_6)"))
 (segment (start 107.5 80) (end 106.79 79.29) (width 0.2) (layer "F.Cu") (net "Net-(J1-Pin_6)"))
 (via (at 107.5 80) (size 0.6) (drill 0.3) (layers "F.Cu" "B.Cu") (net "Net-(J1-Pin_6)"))
 (via (at 121 80.5) (size 0.6) (drill 0.3) (layers "F.Cu" "B.Cu") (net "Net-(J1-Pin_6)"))
 (segment (start 121 80.5) (end 108 80.5) (width 0.2) (layer "B.Cu") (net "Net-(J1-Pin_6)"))
 (segment (start 108 80.5) (end 107.5 80) (width 0.2) (layer "B.Cu") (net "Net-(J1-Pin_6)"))
 (segment (start 69.85 104.17) (end 71 105.32) (width 0.2) (layer "F.Cu") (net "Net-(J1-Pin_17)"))
 (segment (start 120 120.7) (end 121.15 121.85) (width 0.2) (layer "F.Cu") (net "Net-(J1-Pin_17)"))
 (segment (start 77.63 101.63) (end 70.523654 101.63) (width 0.2) (layer "F.Cu") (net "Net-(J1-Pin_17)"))
 (segment (start 86.5 110.5) (end 77.63 101.63) (width 0.2) (layer "F.Cu") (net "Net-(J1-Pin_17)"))
 (segment (start 121.15 123.716346) (end 120.476346 124.39) (width 0.2) (layer "F.Cu") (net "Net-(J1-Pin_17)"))
 (segment (start 69.85 102.303654) (end 69.85 104.17) (width 0.2) (layer "F.Cu") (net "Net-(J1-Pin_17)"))
 (segment (start 70.523654 101.63) (end 69.85 102.303654) (width 0.2) (layer "F.Cu") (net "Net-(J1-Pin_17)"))
 (segment (start 106.79 124.39) (end 104 121.6) (width 0.2) (layer "F.Cu") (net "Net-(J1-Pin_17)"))
 (segment (start 120.476346 124.39) (end 106.79 124.39) (width 0.2) (layer "F.Cu") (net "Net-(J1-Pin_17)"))
 (segment (start 121.15 121.85) (end 121.15 123.716346) (width 0.2) (layer "F.Cu") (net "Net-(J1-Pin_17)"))
 (via (at 104 121.6) (size 0.6) (drill 0.3) (layers "F.Cu" "B.Cu") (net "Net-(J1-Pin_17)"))
 (via (at 86.5 110.5) (size 0.6) (drill 0.3) (layers "F.Cu" "B.Cu") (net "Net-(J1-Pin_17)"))
 (segment (start 87 110.5) (end 86.5 110.5) (width 0.2) (layer "B.Cu") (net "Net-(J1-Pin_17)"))
 (segment (start 88.57 112.07) (end 87 110.5) (width 0.2) (layer "B.Cu") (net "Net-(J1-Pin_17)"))
 (segment (start 104 121.6) (end 104 119.193654) (width 0.2) (layer "B.Cu") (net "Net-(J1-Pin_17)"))
 (segment (start 96.876346 112.07) (end 88.57 112.07) (width 0.2) (layer "B.Cu") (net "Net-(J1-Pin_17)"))
 (segment (start 104 119.193654) (end 96.876346 112.07) (width 0.2) (layer "B.Cu") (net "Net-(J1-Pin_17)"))
 (segment (start 122 111.08) (end 122 91) (width 0.2) (layer "F.Cu") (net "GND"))
 (segment (start 117.84 86.84) (end 117.84 71.023654) (width 0.2) (layer "F.Cu") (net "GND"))
 (segment (start 72.27 134.5) (end 71 133.23) (width 0.2) (layer "F.Cu") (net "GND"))
 (segment (start 71 133.23) (end 71 118.02) (width 0.2) (layer "F.Cu") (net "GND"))
 (segment (start 113.39 119.69) (end 120 113.08) (width 0.2) (layer "F.Cu") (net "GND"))
 (segment (start 71 118.02) (end 72.67 119.69) (width 0.2) (layer "F.Cu") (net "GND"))
 (segment (start 122 91) (end 117.84 86.84) (width 0.2) (layer "F.Cu") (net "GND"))
 (segment (start 115.3 70.35) (end 114.15 71.5) (width 0.2) (layer "F.Cu") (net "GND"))
 (segment (start 117.166346 70.35) (end 115.3 70.35) (width 0.2) (layer "F.Cu") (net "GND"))
 (segment (start 72.67 119.69) (end 113.39 119.69) (width 0.2) (layer "F.Cu") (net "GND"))
 (segment (start 117.84 71.023654) (end 117.166346 70.35) (width 0.2) (layer "F.Cu") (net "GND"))
 (segment (start 120 113.08) (end 122 111.08) (width 0.2) (layer "F.Cu") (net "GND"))
 (segment (start 124.31 71.5) (end 121.5 74.31) (width 0.2) (layer "F.Cu") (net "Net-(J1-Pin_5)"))
 (segment (start 107 78) (end 105.75 76.75) (width 0.2) (layer "F.Cu") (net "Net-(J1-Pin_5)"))
 (segment (start 121.5 74.31) (end 121.5 79) (width 0.2) (layer "F.Cu") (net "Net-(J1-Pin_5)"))
 (segment (start 72.91 76.75) (end 71 74.84) (width 0.2) (layer "F.Cu") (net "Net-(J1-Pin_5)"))
 (segment (start 105.75 76.75) (end 72.91 76.75) (width 0.2) (layer "F.Cu") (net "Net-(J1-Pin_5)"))
 (via (at 107 78) (size 0.6) (drill 0.3) (layers "F.Cu" "B.Cu") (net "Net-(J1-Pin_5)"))
 (via (at 121.5 79) (size 0.6) (drill 0.3) (layers "F.Cu" "B.Cu") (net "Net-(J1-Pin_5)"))
 (segment (start 109.5 78) (end 107 78) (width 0.2) (layer "B.Cu") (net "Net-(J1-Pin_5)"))
 (segment (start 121.5 79) (end 110.5 79) (width 0.2) (layer "B.Cu") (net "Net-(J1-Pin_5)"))
 (segment (start 110.5 79) (end 109.5 78) (width 0.2) (layer "B.Cu") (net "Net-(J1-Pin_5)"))
 (segment (start 105.28 125.78) (end 102 122.5) (width 0.2) (layer "F.Cu") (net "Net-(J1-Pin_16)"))
 (segment (start 85.5 110.97) (end 79.19 110.97) (width 0.2) (layer "F.Cu") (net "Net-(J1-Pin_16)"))
 (segment (start 86 111.47) (end 85.5 110.97) (width 0.2) (layer "F.Cu") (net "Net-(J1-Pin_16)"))
 (segment (start 120 125.78) (end 105.28 125.78) (width 0.2) (layer "F.Cu") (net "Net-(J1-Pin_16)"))
 (segment (start 79.19 110.97) (end 71 102.78) (width 0.2) (layer "F.Cu") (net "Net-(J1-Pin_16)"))
 (via (at 86 111.47) (size 0.6) (drill 0.3) (layers "F.Cu" "B.Cu") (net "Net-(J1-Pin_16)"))
 (via (at 102 122.5) (size 0.6) (drill 0.3) (layers "F.Cu" "B.Cu") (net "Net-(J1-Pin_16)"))
 (segment (start 102 122.5) (end 97.03 122.5) (width 0.2) (layer "B.Cu") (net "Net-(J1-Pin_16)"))
 (segment (start 97.03 122.5) (end 86 111.47) (width 0.2) (layer "B.Cu") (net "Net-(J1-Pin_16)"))
 (segment (start 93.61 114.61) (end 92 113) (width 0.2) (layer "F.Cu") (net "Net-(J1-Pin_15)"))
 (segment (start 88 109.5) (end 78.74 100.24) (width 0.2) (layer "F.Cu") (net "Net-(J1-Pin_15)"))
 (segment (start 78.74 100.24) (end 71 100.24) (width 0.2) (layer "F.Cu") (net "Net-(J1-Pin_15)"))
 (segment (start 115.93 114.61) (end 93.61 114.61) (width 0.2) (layer "F.Cu") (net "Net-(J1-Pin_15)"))
 (segment (start 88 110.47) (end 88 109.5) (width 0.2) (layer "F.Cu") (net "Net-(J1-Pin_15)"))
 (segment (start 120 110.54) (end 115.93 114.61) (width 0.2) (layer "F.Cu") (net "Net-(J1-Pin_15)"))
 (segment (start 87 111.47) (end 88 110.47) (width 0.2) (layer "F.Cu") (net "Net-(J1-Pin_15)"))
 (via (at 92 113) (size 0.6) (drill 0.3) (layers "F.Cu" "B.Cu") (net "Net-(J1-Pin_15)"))
 (via (at 87 111.47) (size 0.6) (drill 0.3) (layers "F.Cu" "B.Cu") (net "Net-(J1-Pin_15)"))
 (segment (start 92 113) (end 88.53 113) (width 0.2) (layer "B.Cu") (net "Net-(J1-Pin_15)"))
 (segment (start 88.53 113) (end 87 111.47) (width 0.2) (layer "B.Cu") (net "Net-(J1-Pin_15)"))
 (segment (start 72.67 73.97) (end 71 72.3) (width 0.2) (layer "F.Cu") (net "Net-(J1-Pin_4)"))
 (segment (start 126.85 73.15) (end 122.5 77.5) (width 0.2) (layer "F.Cu") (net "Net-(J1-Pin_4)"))
 (segment (start 102.97 73.97) (end 72.67 73.97) (width 0.2) (layer "F.Cu") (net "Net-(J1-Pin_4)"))
 (segment (start 126.85 71.5) (end 126.85 73.15) (width 0.2) (layer "F.Cu") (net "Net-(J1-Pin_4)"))
 (segment (start 103.5 74.5) (end 102.97 73.97) (width 0.2) (layer "F.Cu") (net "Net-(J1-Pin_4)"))
 (via (at 122.5 77.5) (size 0.6) (drill 0.3) (layers "F.Cu" "B.Cu") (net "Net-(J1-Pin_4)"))
 (via (at 103.5 74.5) (size 0.6) (drill 0.3) (layers "F.Cu" "B.Cu") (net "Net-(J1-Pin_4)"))
 (segment (start 122 77) (end 106 77) (width 0.2) (layer "B.Cu") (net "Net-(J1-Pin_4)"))
 (segment (start 122.5 77.5) (end 122 77) (width 0.2) (layer "B.Cu") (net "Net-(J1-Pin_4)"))
 (segment (start 106 77) (end 103.5 74.5) (width 0.2) (layer "B.Cu") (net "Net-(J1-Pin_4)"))
 (segment (start 99.34 91) (end 96.4 88.06) (width 0.2) (layer "F.Cu") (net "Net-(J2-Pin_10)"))
 (segment (start 116.92 91) (end 99.34 91) (width 0.2) (layer "F.Cu") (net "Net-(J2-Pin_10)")))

